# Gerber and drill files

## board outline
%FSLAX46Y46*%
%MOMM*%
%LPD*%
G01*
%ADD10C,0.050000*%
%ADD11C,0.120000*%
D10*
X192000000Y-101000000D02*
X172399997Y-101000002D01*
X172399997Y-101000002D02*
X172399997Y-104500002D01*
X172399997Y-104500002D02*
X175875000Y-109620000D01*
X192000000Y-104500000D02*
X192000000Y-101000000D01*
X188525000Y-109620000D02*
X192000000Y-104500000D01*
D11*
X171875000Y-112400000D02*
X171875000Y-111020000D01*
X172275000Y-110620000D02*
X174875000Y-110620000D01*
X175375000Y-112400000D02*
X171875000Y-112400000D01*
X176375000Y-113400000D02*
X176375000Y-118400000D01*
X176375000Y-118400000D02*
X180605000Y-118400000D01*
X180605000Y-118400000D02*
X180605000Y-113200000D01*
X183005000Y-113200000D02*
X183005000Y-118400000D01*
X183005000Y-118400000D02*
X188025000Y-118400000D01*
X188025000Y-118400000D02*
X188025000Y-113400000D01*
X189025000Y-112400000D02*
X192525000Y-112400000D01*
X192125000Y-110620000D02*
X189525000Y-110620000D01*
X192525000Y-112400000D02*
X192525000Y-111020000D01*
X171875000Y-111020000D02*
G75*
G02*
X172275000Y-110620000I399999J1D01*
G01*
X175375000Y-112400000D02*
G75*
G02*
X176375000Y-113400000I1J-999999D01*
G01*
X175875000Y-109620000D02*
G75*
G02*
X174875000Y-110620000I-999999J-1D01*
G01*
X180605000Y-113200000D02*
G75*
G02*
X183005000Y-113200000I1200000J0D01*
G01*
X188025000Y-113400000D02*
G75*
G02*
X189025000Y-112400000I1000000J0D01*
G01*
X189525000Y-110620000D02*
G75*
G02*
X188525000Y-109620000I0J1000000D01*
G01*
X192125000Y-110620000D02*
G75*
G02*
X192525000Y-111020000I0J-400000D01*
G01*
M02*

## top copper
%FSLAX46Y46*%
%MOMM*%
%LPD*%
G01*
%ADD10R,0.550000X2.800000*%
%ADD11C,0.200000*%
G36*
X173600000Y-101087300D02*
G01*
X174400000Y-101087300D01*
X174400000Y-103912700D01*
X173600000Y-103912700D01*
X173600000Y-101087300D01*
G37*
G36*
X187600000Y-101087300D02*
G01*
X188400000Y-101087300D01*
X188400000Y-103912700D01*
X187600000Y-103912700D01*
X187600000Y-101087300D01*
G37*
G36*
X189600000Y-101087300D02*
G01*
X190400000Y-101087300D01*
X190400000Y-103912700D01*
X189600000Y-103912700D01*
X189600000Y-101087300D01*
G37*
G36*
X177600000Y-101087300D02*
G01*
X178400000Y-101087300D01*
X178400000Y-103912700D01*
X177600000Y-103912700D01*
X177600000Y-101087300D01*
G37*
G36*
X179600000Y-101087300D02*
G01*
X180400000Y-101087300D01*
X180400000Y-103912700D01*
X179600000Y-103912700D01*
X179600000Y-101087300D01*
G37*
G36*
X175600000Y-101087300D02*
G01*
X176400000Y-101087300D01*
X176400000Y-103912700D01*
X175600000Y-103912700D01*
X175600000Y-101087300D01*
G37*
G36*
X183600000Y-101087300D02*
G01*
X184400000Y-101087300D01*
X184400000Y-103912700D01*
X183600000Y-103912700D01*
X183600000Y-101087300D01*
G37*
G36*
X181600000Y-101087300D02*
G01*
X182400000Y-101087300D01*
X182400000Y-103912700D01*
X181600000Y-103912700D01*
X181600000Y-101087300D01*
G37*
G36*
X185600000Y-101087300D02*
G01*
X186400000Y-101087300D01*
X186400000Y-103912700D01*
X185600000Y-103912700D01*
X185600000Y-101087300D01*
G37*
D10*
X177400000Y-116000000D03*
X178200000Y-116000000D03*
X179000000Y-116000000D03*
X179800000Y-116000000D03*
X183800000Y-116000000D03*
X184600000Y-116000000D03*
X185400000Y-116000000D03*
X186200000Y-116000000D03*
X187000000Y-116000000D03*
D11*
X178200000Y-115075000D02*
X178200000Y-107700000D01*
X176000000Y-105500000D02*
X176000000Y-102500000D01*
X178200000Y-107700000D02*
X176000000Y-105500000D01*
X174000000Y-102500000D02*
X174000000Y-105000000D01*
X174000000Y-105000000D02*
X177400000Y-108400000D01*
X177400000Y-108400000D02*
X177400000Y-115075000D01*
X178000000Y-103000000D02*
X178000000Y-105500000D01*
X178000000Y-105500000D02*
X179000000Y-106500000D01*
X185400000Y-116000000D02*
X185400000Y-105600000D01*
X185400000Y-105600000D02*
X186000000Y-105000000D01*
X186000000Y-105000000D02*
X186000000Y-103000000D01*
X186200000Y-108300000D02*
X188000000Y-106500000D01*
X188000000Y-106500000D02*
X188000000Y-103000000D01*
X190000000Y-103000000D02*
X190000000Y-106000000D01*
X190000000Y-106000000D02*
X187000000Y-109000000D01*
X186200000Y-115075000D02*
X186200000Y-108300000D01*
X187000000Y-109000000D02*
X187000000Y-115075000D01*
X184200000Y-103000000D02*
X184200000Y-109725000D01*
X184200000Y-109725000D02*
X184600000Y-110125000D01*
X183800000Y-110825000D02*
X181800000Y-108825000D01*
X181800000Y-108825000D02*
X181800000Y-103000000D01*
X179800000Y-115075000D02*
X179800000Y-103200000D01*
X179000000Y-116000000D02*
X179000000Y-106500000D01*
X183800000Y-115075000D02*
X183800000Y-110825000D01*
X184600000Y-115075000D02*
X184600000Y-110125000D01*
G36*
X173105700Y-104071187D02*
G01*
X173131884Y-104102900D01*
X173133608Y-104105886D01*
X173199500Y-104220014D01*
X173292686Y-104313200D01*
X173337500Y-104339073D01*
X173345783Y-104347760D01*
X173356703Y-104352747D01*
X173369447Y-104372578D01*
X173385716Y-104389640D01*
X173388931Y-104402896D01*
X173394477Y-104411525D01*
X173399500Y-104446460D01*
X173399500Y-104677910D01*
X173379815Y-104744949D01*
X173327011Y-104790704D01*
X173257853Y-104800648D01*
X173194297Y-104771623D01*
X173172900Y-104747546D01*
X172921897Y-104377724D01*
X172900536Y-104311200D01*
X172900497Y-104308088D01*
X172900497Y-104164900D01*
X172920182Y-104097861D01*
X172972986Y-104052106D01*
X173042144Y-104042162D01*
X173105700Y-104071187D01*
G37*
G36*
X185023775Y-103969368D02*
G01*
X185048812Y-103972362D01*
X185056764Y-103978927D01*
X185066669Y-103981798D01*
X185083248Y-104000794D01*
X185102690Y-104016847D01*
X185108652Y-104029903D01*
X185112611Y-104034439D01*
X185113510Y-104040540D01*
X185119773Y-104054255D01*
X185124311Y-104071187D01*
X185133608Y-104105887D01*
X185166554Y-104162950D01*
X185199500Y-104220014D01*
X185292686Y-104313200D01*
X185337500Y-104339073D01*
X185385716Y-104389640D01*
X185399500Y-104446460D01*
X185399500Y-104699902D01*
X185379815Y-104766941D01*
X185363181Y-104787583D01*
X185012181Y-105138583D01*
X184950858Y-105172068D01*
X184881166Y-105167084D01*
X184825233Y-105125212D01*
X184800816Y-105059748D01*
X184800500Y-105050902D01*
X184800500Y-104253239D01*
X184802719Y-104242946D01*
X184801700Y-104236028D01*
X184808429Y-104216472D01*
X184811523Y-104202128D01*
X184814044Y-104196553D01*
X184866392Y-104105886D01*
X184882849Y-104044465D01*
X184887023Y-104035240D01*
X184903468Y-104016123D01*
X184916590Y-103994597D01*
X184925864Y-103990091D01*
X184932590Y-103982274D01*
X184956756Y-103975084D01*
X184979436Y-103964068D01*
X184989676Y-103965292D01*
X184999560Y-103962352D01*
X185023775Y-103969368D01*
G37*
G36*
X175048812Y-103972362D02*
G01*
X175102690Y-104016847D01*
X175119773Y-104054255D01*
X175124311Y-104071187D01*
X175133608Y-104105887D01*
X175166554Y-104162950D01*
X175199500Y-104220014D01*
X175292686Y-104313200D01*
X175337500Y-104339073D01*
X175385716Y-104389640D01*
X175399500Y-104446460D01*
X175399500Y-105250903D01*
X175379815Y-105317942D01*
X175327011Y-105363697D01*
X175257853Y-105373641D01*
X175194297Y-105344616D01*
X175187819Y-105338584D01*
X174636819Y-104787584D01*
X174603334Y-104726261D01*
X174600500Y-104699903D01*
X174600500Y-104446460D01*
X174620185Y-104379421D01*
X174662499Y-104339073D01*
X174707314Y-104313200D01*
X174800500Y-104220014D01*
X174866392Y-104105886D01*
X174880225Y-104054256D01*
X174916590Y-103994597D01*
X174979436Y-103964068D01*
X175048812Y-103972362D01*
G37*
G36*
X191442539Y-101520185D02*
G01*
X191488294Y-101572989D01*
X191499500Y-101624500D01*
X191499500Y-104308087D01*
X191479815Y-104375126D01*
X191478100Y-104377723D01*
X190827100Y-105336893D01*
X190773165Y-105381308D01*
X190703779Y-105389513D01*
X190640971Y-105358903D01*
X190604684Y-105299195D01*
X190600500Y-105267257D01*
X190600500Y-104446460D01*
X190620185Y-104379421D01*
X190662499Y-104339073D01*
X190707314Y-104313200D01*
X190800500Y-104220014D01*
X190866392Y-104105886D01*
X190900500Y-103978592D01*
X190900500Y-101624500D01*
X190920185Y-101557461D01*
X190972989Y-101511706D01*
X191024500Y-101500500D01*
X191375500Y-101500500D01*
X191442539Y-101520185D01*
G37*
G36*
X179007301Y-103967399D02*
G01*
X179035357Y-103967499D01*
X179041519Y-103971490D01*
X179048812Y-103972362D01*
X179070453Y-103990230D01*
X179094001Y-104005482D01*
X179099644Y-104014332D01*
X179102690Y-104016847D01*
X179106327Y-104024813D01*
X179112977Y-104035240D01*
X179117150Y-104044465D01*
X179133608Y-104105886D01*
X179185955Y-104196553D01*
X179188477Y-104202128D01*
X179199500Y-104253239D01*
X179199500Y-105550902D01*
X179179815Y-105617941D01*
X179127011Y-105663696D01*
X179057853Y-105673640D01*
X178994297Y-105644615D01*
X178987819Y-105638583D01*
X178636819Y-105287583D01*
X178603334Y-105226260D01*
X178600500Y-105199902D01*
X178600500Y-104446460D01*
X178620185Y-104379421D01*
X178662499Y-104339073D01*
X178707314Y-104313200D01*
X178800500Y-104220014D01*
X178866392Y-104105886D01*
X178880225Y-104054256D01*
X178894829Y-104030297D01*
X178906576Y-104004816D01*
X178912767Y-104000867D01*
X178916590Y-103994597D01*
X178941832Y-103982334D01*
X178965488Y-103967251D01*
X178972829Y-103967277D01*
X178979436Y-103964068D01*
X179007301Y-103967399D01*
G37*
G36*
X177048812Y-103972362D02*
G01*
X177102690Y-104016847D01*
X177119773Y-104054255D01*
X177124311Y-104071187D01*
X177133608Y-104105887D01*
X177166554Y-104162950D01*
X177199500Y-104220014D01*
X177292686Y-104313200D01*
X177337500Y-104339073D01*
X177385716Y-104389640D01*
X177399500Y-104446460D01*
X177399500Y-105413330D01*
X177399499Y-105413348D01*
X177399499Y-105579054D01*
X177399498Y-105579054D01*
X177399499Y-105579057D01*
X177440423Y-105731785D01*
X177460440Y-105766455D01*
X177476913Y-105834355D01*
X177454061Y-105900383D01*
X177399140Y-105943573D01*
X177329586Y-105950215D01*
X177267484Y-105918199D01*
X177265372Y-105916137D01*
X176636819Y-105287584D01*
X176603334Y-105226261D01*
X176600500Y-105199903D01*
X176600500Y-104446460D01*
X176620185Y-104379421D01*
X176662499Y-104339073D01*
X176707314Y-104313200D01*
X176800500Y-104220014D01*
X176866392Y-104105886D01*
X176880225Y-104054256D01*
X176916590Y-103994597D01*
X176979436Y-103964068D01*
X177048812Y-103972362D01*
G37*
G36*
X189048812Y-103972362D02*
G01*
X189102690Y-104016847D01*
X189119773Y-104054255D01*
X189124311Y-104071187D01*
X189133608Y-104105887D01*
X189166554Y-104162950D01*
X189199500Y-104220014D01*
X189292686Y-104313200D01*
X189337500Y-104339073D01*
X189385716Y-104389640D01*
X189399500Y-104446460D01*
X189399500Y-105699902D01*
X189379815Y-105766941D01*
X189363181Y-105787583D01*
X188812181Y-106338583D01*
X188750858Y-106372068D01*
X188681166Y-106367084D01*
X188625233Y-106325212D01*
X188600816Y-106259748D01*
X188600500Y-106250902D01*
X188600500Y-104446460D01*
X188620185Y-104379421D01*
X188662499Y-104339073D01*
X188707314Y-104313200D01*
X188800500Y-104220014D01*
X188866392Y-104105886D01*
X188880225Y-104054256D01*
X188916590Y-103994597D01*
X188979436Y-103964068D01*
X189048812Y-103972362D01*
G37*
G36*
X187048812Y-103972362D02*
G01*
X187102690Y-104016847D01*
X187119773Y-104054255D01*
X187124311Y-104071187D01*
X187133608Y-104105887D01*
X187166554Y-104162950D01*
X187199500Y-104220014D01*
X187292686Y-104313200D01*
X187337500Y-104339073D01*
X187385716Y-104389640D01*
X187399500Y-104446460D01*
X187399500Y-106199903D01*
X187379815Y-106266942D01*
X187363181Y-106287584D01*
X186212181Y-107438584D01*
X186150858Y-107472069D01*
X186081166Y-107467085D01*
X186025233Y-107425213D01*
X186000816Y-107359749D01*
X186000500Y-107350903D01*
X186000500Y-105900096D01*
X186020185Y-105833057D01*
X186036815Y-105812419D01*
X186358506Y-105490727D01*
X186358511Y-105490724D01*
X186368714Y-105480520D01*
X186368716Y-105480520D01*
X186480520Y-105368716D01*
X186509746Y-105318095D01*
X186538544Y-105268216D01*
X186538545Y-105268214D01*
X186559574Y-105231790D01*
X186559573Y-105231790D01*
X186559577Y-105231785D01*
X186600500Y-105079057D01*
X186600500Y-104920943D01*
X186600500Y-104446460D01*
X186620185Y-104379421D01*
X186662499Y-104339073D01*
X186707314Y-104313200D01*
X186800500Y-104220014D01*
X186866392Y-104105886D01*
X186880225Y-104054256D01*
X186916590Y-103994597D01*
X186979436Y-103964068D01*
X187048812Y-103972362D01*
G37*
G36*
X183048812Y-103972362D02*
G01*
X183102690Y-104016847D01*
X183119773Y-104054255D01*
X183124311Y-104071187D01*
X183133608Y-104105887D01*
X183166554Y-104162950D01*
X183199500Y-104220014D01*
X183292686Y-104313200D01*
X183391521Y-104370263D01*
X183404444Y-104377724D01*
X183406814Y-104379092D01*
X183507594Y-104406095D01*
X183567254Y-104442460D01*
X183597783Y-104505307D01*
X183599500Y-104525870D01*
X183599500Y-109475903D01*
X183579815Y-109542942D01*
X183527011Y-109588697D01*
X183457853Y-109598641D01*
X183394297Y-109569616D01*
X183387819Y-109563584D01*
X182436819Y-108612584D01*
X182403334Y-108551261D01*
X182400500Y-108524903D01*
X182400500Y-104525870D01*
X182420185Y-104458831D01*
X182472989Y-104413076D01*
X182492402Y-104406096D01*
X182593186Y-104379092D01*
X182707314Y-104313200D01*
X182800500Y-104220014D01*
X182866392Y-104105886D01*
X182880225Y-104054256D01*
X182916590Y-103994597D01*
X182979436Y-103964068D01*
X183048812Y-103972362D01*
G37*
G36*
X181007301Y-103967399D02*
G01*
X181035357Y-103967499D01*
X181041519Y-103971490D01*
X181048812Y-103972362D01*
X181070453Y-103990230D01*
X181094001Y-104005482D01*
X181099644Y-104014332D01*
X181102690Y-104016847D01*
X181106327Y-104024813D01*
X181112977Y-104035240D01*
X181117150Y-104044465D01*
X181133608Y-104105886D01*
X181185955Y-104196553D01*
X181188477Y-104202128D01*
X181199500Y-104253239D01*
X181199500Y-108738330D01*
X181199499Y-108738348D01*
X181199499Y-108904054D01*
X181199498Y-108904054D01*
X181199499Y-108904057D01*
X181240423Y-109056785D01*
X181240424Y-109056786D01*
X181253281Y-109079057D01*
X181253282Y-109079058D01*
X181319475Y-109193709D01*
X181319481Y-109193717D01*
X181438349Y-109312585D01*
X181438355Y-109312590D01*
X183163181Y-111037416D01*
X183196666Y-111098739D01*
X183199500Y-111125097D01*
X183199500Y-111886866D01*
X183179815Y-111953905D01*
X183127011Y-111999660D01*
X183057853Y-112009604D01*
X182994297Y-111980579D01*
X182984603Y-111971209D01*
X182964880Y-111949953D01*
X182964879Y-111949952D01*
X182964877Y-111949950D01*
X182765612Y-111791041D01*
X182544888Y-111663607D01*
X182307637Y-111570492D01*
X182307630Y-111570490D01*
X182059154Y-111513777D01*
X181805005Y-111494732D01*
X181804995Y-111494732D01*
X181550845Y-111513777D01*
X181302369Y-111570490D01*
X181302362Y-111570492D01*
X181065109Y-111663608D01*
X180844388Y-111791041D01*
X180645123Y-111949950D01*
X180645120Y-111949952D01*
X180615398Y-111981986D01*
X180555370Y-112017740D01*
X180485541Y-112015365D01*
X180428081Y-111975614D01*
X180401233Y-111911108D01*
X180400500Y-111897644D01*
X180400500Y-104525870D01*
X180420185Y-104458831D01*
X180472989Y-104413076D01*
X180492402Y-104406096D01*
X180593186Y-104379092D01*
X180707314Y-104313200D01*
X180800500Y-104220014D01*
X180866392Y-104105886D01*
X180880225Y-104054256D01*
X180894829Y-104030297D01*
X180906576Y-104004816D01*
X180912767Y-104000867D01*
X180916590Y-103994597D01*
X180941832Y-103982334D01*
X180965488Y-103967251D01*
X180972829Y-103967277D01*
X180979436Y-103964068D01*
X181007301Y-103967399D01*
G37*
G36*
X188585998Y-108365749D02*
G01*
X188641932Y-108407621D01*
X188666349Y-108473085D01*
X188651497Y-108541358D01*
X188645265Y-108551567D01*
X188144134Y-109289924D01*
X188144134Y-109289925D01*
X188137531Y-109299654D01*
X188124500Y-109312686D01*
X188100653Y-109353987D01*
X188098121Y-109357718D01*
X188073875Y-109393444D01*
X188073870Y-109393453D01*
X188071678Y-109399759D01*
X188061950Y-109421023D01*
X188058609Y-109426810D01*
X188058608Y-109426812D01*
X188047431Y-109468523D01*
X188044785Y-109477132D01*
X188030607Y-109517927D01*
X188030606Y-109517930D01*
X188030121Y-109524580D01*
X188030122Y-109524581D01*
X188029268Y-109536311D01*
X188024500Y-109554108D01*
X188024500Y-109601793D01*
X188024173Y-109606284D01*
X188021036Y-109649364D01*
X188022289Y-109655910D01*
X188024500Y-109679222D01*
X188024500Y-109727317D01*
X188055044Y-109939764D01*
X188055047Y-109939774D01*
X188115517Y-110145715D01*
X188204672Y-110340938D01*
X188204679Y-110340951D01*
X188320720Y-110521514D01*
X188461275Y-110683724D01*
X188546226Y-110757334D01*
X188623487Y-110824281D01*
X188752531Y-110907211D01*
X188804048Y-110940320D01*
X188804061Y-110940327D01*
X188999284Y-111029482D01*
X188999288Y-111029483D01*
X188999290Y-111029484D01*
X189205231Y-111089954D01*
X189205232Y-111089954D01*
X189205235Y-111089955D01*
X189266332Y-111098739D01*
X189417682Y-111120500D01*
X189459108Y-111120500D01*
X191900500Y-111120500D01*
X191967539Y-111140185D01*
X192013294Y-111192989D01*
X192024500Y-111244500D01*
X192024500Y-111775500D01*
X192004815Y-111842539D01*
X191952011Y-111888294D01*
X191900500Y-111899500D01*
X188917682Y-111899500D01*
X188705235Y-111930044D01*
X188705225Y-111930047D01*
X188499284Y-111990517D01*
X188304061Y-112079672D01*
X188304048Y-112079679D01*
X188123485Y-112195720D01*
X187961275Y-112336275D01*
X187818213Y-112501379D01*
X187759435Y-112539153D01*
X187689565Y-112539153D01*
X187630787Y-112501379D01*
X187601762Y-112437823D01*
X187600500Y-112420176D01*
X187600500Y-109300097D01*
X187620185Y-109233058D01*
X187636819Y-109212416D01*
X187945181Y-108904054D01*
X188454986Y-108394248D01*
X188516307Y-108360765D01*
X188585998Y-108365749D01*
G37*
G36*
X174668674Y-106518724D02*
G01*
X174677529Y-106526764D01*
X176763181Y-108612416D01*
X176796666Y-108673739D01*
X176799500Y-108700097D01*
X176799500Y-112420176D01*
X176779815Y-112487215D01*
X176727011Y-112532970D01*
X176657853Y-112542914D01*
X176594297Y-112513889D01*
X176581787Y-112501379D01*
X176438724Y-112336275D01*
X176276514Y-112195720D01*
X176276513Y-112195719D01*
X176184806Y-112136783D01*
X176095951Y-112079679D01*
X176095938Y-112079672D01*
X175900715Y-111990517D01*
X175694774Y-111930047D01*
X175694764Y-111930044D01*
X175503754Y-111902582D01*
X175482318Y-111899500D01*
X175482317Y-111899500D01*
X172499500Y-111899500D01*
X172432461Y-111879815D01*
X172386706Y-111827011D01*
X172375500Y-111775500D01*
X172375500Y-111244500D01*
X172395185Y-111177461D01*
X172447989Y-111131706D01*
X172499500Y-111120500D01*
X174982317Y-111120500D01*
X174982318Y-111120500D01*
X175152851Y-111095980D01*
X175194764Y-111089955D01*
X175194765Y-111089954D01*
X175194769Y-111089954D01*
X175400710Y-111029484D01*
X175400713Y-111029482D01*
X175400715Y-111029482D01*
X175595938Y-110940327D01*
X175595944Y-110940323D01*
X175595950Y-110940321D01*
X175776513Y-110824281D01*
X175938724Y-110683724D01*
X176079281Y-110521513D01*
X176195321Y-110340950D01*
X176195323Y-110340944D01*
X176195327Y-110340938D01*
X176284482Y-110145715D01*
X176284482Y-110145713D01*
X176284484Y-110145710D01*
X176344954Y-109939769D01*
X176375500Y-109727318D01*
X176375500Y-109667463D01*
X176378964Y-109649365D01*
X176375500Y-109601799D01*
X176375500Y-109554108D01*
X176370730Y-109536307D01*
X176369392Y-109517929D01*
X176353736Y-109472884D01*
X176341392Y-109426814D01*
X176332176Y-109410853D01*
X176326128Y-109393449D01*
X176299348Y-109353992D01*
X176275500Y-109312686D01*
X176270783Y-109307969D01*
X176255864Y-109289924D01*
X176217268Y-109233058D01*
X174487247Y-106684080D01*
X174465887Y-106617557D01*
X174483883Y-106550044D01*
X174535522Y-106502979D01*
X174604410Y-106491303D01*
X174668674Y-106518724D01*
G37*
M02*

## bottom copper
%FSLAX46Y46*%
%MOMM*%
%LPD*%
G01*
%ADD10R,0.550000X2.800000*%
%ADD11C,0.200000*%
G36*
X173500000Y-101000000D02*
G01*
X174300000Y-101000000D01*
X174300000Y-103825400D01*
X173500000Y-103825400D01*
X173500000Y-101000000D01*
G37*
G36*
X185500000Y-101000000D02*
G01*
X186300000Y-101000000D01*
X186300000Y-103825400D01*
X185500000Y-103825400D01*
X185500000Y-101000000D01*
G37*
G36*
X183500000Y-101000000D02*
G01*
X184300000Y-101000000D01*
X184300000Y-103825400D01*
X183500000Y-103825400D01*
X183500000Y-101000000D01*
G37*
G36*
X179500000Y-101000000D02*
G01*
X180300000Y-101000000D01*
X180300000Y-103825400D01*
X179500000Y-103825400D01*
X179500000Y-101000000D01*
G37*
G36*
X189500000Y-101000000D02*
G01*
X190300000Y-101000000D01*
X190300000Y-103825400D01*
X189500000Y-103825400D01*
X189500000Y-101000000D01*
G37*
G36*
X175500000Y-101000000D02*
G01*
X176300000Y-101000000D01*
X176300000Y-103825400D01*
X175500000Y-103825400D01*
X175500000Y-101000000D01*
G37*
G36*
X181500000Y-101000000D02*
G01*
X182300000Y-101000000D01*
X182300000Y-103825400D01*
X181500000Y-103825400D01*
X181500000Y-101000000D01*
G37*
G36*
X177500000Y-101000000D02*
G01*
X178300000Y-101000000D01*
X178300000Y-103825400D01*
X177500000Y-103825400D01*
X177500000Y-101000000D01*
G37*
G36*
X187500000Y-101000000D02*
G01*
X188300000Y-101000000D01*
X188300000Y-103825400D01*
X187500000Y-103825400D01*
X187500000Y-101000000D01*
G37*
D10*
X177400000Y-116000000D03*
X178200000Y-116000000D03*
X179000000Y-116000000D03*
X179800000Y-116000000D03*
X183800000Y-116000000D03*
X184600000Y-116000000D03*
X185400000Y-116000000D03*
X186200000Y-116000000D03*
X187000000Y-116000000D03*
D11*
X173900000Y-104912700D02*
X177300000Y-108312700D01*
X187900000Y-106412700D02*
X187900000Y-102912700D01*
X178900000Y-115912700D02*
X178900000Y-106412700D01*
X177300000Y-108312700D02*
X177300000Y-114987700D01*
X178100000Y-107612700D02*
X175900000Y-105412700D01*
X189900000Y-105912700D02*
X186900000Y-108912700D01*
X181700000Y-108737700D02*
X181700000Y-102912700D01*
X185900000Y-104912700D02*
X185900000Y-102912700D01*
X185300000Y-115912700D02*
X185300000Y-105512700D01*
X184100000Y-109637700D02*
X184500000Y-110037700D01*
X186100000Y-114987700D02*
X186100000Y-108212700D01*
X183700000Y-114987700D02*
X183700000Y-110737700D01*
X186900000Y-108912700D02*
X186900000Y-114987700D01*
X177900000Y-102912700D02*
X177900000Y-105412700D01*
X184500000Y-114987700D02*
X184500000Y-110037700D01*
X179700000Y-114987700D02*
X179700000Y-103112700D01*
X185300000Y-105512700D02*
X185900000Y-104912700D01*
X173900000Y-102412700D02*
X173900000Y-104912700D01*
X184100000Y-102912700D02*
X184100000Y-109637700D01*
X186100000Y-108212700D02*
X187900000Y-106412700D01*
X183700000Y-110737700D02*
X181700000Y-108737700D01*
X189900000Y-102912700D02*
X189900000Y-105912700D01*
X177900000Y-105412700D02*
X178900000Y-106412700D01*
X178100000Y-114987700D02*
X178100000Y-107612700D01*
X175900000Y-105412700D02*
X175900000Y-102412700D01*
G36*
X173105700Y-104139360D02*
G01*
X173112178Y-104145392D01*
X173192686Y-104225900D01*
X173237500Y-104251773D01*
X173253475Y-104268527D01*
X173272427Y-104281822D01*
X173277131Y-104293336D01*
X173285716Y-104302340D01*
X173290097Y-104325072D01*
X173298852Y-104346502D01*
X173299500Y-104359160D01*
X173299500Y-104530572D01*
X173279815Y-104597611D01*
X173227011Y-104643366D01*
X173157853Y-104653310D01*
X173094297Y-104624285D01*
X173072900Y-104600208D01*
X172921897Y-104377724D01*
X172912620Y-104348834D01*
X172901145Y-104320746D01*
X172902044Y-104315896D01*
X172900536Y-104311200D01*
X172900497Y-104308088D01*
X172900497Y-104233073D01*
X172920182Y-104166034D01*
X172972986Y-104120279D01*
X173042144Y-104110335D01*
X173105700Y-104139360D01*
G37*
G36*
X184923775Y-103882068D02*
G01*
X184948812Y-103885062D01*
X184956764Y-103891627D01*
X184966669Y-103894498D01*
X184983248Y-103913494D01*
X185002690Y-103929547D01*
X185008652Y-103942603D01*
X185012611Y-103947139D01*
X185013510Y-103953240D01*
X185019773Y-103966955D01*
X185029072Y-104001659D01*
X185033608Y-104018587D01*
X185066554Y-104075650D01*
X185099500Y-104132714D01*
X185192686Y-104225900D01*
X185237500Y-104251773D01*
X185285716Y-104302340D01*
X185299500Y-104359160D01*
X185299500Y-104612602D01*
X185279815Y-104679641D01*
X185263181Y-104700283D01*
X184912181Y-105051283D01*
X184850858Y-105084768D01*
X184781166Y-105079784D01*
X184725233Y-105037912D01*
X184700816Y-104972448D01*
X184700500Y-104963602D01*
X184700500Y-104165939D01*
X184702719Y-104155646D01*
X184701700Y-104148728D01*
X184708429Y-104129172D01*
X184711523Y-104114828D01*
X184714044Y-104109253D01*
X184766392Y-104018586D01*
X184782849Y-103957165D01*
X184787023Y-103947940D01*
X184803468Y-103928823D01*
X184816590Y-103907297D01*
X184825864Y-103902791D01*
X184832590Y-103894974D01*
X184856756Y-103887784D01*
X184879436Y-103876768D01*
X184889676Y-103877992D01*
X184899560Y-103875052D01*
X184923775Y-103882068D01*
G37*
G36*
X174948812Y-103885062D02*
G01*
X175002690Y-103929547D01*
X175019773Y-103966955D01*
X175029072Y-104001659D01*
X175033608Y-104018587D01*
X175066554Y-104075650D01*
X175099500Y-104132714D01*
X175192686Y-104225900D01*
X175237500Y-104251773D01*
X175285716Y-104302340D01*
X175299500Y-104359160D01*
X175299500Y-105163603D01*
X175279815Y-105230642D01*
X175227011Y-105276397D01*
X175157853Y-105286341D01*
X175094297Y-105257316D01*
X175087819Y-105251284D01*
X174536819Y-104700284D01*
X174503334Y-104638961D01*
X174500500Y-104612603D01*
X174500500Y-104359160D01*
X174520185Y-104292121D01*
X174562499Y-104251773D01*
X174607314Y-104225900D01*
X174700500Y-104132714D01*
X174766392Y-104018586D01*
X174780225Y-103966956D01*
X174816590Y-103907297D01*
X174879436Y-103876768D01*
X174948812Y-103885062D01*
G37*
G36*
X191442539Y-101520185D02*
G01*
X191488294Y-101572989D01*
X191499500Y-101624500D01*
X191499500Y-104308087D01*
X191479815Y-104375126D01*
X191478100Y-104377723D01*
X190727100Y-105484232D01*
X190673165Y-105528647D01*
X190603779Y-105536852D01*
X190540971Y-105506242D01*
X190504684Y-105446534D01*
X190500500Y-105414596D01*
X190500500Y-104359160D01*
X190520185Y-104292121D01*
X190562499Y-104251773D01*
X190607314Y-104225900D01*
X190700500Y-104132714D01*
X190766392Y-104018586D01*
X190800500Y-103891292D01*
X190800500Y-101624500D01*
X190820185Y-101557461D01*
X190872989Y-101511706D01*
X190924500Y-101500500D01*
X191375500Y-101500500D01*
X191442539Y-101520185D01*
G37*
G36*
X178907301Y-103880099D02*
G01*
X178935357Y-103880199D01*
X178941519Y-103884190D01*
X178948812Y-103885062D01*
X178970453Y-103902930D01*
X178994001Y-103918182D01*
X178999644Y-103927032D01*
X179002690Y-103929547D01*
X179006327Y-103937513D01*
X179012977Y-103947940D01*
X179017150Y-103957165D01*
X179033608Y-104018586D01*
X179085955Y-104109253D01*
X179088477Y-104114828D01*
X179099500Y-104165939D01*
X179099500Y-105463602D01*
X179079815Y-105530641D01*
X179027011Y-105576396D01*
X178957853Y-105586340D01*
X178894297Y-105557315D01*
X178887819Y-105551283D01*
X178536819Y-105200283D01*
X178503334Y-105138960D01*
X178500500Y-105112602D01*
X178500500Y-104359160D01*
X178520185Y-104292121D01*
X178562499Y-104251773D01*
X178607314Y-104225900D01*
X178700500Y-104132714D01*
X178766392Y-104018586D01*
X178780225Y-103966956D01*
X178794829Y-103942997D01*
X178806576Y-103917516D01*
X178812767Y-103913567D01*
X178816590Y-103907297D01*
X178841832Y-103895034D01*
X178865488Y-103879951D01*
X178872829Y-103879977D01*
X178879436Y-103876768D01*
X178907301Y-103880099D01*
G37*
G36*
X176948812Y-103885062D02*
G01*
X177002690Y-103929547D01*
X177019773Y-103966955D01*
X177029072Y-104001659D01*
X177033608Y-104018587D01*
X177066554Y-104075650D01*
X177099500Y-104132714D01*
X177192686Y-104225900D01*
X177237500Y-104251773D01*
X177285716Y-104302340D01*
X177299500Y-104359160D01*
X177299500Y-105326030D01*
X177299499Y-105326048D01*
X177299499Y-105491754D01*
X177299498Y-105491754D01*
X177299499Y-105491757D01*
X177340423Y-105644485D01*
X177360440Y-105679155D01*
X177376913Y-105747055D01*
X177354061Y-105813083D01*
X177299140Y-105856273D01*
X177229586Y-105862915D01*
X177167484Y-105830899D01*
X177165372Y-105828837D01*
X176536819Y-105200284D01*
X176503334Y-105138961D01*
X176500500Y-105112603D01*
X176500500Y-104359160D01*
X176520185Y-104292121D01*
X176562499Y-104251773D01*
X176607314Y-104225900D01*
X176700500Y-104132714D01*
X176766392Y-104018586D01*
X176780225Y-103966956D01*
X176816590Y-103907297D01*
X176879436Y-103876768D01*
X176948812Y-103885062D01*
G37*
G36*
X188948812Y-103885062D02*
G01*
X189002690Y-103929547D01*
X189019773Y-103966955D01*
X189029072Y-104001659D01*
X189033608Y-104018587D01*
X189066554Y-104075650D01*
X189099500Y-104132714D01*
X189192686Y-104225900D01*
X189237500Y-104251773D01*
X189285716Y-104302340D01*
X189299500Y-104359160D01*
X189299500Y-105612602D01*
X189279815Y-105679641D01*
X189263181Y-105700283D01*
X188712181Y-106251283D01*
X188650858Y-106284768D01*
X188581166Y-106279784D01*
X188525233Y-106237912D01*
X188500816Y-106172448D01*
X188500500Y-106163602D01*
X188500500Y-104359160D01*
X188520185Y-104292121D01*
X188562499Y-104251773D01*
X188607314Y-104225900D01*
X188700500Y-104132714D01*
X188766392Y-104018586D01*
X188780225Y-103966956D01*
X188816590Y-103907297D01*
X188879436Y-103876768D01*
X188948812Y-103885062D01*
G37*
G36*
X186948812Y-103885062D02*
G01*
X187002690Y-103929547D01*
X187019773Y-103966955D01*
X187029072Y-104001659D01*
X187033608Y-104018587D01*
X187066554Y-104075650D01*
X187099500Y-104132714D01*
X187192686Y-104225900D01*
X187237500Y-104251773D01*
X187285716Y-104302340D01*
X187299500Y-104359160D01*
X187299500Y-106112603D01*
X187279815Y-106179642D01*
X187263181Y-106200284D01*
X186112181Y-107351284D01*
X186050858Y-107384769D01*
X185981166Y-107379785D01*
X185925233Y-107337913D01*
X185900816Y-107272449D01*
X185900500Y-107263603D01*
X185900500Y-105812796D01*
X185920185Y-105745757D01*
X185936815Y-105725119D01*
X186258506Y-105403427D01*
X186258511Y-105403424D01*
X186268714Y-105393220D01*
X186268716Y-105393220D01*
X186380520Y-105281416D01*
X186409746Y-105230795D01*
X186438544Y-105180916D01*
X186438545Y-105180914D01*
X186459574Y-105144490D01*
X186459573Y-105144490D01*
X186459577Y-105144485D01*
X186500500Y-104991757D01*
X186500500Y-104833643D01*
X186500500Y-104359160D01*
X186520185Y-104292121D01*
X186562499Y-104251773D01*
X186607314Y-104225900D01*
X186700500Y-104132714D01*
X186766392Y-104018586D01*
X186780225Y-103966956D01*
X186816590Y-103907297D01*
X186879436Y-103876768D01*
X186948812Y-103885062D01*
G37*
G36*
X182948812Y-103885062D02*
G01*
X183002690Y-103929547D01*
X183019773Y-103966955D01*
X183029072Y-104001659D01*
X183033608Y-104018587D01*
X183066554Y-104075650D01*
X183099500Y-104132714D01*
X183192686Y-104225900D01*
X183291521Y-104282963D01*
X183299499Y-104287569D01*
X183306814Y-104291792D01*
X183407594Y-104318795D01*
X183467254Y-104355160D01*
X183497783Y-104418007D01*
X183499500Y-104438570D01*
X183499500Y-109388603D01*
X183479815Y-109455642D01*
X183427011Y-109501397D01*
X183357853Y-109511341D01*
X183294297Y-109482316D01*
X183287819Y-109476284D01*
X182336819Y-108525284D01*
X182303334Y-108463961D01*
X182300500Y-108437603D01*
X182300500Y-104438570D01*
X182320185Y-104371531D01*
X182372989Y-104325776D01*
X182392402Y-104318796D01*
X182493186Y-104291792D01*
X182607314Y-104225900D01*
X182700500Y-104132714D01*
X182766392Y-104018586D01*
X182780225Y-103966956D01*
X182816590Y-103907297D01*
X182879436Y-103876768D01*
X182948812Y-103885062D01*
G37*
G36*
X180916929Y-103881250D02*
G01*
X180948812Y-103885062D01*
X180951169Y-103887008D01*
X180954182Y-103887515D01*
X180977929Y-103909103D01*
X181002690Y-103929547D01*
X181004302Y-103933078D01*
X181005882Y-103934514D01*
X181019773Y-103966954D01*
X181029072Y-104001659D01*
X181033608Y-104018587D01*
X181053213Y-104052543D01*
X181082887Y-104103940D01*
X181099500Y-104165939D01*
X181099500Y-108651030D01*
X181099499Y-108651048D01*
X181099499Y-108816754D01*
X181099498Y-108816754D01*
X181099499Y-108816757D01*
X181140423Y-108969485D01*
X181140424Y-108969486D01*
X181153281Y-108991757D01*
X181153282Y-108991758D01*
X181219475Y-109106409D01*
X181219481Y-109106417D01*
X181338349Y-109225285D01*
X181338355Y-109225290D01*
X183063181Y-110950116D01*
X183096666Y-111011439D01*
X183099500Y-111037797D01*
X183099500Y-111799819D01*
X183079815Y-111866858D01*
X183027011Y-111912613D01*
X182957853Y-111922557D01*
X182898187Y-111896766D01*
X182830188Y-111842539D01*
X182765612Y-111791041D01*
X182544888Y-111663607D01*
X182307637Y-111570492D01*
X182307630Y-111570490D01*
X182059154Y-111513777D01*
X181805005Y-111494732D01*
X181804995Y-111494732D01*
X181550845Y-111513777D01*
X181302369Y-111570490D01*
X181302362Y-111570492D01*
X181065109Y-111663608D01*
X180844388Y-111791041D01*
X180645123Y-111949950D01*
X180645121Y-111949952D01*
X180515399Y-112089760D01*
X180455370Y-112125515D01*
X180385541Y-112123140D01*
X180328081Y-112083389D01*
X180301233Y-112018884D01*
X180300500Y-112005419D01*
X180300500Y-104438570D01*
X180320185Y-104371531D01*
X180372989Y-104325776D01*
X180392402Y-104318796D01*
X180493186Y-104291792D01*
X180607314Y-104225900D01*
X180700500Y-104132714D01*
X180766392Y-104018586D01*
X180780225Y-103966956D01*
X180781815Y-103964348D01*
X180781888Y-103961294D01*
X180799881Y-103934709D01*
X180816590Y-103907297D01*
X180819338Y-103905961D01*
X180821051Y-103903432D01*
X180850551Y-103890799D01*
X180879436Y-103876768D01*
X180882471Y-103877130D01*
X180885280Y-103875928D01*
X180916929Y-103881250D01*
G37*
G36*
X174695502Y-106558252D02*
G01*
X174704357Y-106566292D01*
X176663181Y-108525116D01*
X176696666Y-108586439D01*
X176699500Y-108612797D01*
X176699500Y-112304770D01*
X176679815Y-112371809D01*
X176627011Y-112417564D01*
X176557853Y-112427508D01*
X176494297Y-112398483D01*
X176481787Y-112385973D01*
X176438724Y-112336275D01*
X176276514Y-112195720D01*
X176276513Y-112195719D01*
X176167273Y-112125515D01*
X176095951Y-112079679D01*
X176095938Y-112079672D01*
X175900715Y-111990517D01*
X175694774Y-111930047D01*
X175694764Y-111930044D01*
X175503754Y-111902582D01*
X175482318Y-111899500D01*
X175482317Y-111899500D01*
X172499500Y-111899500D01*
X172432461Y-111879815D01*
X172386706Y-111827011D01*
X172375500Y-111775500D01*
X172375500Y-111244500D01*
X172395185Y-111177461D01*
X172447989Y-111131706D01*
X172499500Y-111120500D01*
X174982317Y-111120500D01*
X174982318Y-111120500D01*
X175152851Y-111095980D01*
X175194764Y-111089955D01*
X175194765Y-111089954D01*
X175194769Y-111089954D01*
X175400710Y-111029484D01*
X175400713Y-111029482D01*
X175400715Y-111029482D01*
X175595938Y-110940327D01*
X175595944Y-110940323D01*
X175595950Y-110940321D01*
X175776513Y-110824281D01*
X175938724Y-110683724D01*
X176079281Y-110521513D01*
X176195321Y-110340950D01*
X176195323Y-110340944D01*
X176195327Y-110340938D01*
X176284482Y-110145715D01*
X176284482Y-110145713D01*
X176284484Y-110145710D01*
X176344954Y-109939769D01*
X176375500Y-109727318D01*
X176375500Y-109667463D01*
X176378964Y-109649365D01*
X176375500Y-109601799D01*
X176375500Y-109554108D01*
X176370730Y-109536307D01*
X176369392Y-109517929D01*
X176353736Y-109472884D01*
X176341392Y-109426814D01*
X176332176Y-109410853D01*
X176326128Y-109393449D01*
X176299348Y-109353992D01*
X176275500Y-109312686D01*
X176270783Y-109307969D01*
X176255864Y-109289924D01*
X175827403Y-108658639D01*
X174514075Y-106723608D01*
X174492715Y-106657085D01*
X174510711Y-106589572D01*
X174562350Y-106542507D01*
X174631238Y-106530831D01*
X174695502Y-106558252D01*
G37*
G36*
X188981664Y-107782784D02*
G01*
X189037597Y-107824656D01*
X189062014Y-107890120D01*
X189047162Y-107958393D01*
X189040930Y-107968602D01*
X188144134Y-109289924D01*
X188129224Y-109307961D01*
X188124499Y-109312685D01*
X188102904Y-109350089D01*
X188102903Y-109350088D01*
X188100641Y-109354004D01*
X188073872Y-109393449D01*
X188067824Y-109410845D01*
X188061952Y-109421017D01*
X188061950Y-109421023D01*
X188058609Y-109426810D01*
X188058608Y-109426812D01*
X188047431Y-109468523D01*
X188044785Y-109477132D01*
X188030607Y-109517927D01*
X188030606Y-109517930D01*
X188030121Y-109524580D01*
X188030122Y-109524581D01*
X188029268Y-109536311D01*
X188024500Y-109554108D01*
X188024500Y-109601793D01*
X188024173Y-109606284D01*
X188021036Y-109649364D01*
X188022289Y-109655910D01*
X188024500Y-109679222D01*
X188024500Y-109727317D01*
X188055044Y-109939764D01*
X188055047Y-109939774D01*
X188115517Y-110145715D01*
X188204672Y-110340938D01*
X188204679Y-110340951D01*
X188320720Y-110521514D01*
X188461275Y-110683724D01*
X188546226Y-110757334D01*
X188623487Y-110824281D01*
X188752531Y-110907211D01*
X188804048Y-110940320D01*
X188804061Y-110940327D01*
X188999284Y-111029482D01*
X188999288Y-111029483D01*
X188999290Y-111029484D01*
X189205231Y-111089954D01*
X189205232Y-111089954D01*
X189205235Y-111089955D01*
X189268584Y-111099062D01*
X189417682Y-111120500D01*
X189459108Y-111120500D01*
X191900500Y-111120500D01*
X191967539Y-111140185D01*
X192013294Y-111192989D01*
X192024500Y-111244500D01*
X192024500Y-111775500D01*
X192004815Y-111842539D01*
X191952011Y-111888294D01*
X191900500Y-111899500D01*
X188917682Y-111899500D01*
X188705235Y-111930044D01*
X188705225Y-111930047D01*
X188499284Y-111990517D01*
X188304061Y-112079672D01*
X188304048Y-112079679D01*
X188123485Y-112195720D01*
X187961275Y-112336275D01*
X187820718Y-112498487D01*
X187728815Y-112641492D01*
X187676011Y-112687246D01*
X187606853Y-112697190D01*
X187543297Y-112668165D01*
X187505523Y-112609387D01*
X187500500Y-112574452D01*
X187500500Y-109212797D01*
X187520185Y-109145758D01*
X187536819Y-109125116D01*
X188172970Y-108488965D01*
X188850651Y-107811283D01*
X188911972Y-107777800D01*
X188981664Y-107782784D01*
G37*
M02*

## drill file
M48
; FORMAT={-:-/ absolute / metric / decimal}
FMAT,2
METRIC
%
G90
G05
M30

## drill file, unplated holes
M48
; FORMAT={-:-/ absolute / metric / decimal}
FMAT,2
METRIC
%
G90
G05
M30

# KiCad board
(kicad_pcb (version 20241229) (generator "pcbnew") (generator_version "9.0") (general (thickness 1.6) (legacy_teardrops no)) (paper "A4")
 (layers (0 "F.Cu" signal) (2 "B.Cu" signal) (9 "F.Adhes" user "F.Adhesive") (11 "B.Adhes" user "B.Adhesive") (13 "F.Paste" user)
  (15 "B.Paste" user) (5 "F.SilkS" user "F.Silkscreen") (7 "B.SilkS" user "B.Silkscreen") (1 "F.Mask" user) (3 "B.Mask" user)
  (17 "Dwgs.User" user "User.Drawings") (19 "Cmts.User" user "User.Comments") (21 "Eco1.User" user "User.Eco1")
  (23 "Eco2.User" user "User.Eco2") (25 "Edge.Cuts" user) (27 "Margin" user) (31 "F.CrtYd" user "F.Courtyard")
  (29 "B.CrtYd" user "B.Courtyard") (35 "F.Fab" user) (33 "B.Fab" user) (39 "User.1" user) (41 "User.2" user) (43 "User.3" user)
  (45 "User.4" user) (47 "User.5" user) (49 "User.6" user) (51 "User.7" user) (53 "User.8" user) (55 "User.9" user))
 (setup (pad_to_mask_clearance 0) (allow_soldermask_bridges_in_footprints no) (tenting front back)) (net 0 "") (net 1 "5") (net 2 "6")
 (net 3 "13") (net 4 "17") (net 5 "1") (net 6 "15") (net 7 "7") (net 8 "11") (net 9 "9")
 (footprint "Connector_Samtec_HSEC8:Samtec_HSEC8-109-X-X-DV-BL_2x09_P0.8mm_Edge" (layer "F.Cu") (at 182.2 118.4)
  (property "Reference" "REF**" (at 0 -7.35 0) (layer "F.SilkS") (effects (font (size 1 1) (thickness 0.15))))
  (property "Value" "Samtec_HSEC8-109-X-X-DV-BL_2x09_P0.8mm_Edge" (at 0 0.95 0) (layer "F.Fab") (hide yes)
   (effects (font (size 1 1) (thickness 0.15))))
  (fp_line (start -10.325 -6) (end -10.325 -7.38) (stroke (width 0.12) (type solid)) (layer "Edge.Cuts"))
  (fp_line (start -9.925 -7.78) (end -7.325 -7.78) (stroke (width 0.12) (type solid)) (layer "Edge.Cuts"))
  (fp_line (start -6.825 -6) (end -10.325 -6) (stroke (width 0.12) (type solid)) (layer "Edge.Cuts"))
  (fp_line (start -5.825 -5) (end -5.825 0) (stroke (width 0.12) (type solid)) (layer "Edge.Cuts"))
  (fp_line (start -5.825 0) (end -1.595 0) (stroke (width 0.12) (type solid)) (layer "Edge.Cuts"))
  (fp_line (start -1.595 0) (end -1.595 -5.2) (stroke (width 0.12) (type solid)) (layer "Edge.Cuts"))
  (fp_line (start 0.805 -5.2) (end 0.805 0) (stroke (width 0.12) (type solid)) (layer "Edge.Cuts"))
  (fp_line (start 0.805 0) (end 5.825 0) (stroke (width 0.12) (type solid)) (layer "Edge.Cuts"))
  (fp_line (start 5.825 0) (end 5.825 -5) (stroke (width 0.12) (type solid)) (layer "Edge.Cuts"))
  (fp_line (start 6.825 -6) (end 10.325 -6) (stroke (width 0.12) (type solid)) (layer "Edge.Cuts"))
  (fp_line (start 9.925 -7.78) (end 7.325 -7.78) (stroke (width 0.12) (type solid)) (layer "Edge.Cuts"))
  (fp_line (start 10.325 -6) (end 10.325 -7.38) (stroke (width 0.12) (type solid)) (layer "Edge.Cuts"))
  (fp_arc (start -10.325 -7.38) (mid -10.207843 -7.662843) (end -9.925 -7.78) (stroke (width 0.12) (type solid)) (layer "Edge.Cuts"))
  (fp_arc (start -6.825 -6) (mid -6.117893 -5.707107) (end -5.825 -5) (stroke (width 0.12) (type solid)) (layer "Edge.Cuts"))
  (fp_arc (start -6.325 -8.78) (mid -6.617893 -8.072893) (end -7.325 -7.78) (stroke (width 0.12) (type solid)) (layer "Edge.Cuts"))
  (fp_arc (start -1.595 -5.2) (mid -0.395 -6.4) (end 0.805 -5.2) (stroke (width 0.12) (type solid)) (layer "Edge.Cuts"))
  (fp_arc (start 5.825 -5) (mid 6.117893 -5.707107) (end 6.825 -6) (stroke (width 0.12) (type solid)) (layer "Edge.Cuts"))
  (fp_arc (start 7.325 -7.78) (mid 6.617893 -8.072893) (end 6.325 -8.78) (stroke (width 0.12) (type solid)) (layer "Edge.Cuts"))
  (fp_arc (start 9.925 -7.78) (mid 10.207843 -7.662843) (end 10.325 -7.38) (stroke (width 0.12) (type solid)) (layer "Edge.Cuts"))
  (pad "1" connect rect (at -4.8 -2.4) (size 0.55 2.8) (layers "F.Cu" "F.Mask"))
  (pad "2" connect rect (at -4.8 -2.4) (size 0.55 2.8) (layers "B.Cu" "B.Mask"))
  (pad "3" connect rect (at -4 -2.4) (size 0.55 2.8) (layers "F.Cu" "F.Mask"))
  (pad "4" connect rect (at -4 -2.4) (size 0.55 2.8) (layers "B.Cu" "B.Mask"))
  (pad "5" connect rect (at -3.2 -2.4) (size 0.55 2.8) (layers "F.Cu" "F.Mask") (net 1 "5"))
  (pad "6" connect rect (at -3.2 -2.4) (size 0.55 2.8) (layers "B.Cu" "B.Mask") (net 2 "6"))
  (pad "7" connect rect (at -2.4 -2.4) (size 0.55 2.8) (layers "F.Cu" "F.Mask"))
  (pad "8" connect rect (at -2.4 -2.4) (size 0.55 2.8) (layers "B.Cu" "B.Mask"))
  (pad "9" connect rect (at 1.6 -2.4) (size 0.55 2.8) (layers "F.Cu" "F.Mask"))
  (pad "10" connect rect (at 1.6 -2.4) (size 0.55 2.8) (layers "B.Cu" "B.Mask"))
  (pad "11" connect rect (at 2.4 -2.4) (size 0.55 2.8) (layers "F.Cu" "F.Mask"))
  (pad "12" connect rect (at 2.4 -2.4) (size 0.55 2.8) (layers "B.Cu" "B.Mask"))
  (pad "13" connect rect (at 3.2 -2.4) (size 0.55 2.8) (layers "F.Cu" "F.Mask") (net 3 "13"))
  (pad "14" connect rect (at 3.2 -2.4) (size 0.55 2.8) (layers "B.Cu" "B.Mask"))
  (pad "15" connect rect (at 4 -2.4) (size 0.55 2.8) (layers "F.Cu" "F.Mask"))
  (pad "16" connect rect (at 4 -2.4) (size 0.55 2.8) (layers "B.Cu" "B.Mask"))
  (pad "17" connect rect (at 4.8 -2.4) (size 0.55 2.8) (layers "F.Cu" "F.Mask") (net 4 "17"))
  (pad "18" connect rect (at 4.8 -2.4) (size 0.55 2.8) (layers "B.Cu" "B.Mask")))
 (gr_rect (start 173.6 101.0873) (end 174.4 103.9127) (stroke (width 0) (type solid)) (fill yes) (layers "F.Cu" "F.Mask") (net 5))
 (gr_rect (start 187.6 101.0873) (end 188.4 103.9127) (stroke (width 0) (type solid)) (fill yes) (layers "F.Cu" "F.Mask") (net 6))
 (gr_rect (start 189.6 101.0873) (end 190.4 103.9127) (stroke (width 0) (type solid)) (fill yes) (layers "F.Cu" "F.Mask") (net 4))
 (gr_rect (start 177.6 101.0873) (end 178.4 103.9127) (stroke (width 0) (type solid)) (fill yes) (layers "F.Cu" "F.Mask") (net 1))
 (gr_rect (start 179.6 101.0873) (end 180.4 103.9127) (stroke (width 0) (type solid)) (fill yes) (layers "F.Cu" "F.Mask") (net 7))
 (gr_rect (start 175.6 101.0873) (end 176.4 103.9127) (stroke (width 0) (type solid)) (fill yes) (layers "F.Cu" "F.Mask") (net 5))
 (gr_rect (start 183.6 101.0873) (end 184.4 103.9127) (stroke (width 0) (type solid)) (fill yes) (layers "F.Cu" "F.Mask") (net 8))
 (gr_rect (start 181.6 101.0873) (end 182.4 103.9127) (stroke (width 0) (type solid)) (fill yes) (layers "F.Cu" "F.Mask") (net 9))
 (gr_rect (start 185.6 101.0873) (end 186.4 103.9127) (stroke (width 0) (type solid)) (fill yes) (layers "F.Cu" "F.Mask") (net 3))
 (gr_rect (start 175.5 101) (end 176.3 103.8254) (stroke (width 0) (type solid)) (fill yes) (layers "B.Cu" "B.Mask") (net 5))
 (gr_rect (start 177.5 101) (end 178.3 103.8254) (stroke (width 0) (type solid)) (fill yes) (layers "B.Cu" "B.Mask") (net 2))
 (gr_rect (start 173.5 101) (end 174.3 103.8254) (stroke (width 0) (type solid)) (fill yes) (layers "B.Cu" "B.Mask") (net 5))
 (gr_rect (start 179.5 101) (end 180.3 103.8254) (stroke (width 0) (type solid)) (fill yes) (layers "B.Cu" "B.Mask") (net 7))
 (gr_rect (start 189.5 101) (end 190.3 103.8254) (stroke (width 0) (type solid)) (fill yes) (layers "B.Cu" "B.Mask") (net 4))
 (gr_rect (start 183.5 101) (end 184.3 103.8254) (stroke (width 0) (type solid)) (fill yes) (layers "B.Cu" "B.Mask") (net 8))
 (gr_rect (start 181.5 101) (end 182.3 103.8254) (stroke (width 0) (type solid)) (fill yes) (layers "B.Cu" "B.Mask") (net 9))
 (gr_rect (start 187.5 101) (end 188.3 103.8254) (stroke (width 0) (type solid)) (fill yes) (layers "B.Cu" "B.Mask") (net 6))
 (gr_rect (start 185.5 101) (end 186.3 103.8254) (stroke (width 0) (type solid)) (fill yes) (layers "B.Cu" "B.Mask") (net 3))
 (gr_line (start 192 101) (end 172.399997 101.000002) (stroke (width 0.05) (type default)) (layer "Edge.Cuts"))
 (gr_line (start 172.399997 104.500002) (end 175.875 109.62) (stroke (width 0.05) (type solid)) (layer "Edge.Cuts"))
 (gr_line (start 172.399997 101.000002) (end 172.399997 104.500002) (stroke (width 0.05) (type default)) (layer "Edge.Cuts"))
 (gr_line (start 192 104.5) (end 192 101) (stroke (width 0.05) (type default)) (layer "Edge.Cuts"))
 (gr_line (start 188.525 109.62) (end 192 104.5) (stroke (width 0.05) (type default)) (layer "Edge.Cuts"))
 (segment (start 178.2 107.7) (end 176 105.5) (width 0.2) (layer "F.Cu") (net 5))
 (segment (start 176 105.5) (end 176 102.5) (width 0.2) (layer "F.Cu") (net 5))
 (segment (start 178.2 115.075) (end 178.2 107.7) (width 0.2) (layer "F.Cu") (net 5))
 (segment (start 177.4 108.4) (end 177.4 115.075) (width 0.2) (layer "F.Cu") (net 5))
 (segment (start 174 102.5) (end 174 105) (width 0.2) (layer "F.Cu") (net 5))
 (segment (start 174 105) (end 177.4 108.4) (width 0.2) (layer "F.Cu") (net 5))
 (segment (start 177.3 108.3127) (end 177.3 114.9877) (width 0.2) (layer "B.Cu") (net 5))
 (segment (start 175.9 105.4127) (end 175.9 102.4127) (width 0.2) (layer "B.Cu") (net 5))
 (segment (start 173.9 102.4127) (end 173.9 104.9127) (width 0.2) (layer "B.Cu") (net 5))
 (segment (start 178.1 114.9877) (end 178.1 107.6127) (width 0.2) (layer "B.Cu") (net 5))
 (segment (start 173.9 104.9127) (end 177.3 108.3127) (width 0.2) (layer "B.Cu") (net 5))
 (segment (start 178.1 107.6127) (end 175.9 105.4127) (width 0.2) (layer "B.Cu") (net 5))
 (segment (start 178 105.5) (end 179 106.5) (width 0.2) (layer "F.Cu") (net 1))
 (segment (start 178 103) (end 178 105.5) (width 0.2) (layer "F.Cu") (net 1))
 (segment (start 179 116) (end 179 106.5) (width 0.2) (layer "F.Cu") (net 1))
 (segment (start 179.8 115.075) (end 179.8 103.2) (width 0.2) (layer "F.Cu") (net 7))
 (segment (start 179.7 114.9877) (end 179.7 103.1127) (width 0.2) (layer "B.Cu") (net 7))
 (segment (start 183.8 115.075) (end 183.8 110.825) (width 0.2) (layer "F.Cu") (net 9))
 (segment (start 183.8 110.825) (end 181.8 108.825) (width 0.2) (layer "F.Cu") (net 9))
 (segment (start 181.8 108.825) (end 181.8 103) (width 0.2) (layer "F.Cu") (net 9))
 (segment (start 183.7 114.9877) (end 183.7 110.7377) (width 0.2) (layer "B.Cu") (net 9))
 (segment (start 181.7 108.7377) (end 181.7 102.9127) (width 0.2) (layer "B.Cu") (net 9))
 (segment (start 183.7 110.7377) (end 181.7 108.7377) (width 0.2) (layer "B.Cu") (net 9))
 (segment (start 184.6 115.075) (end 184.6 110.125) (width 0.2) (layer "F.Cu") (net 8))
 (segment (start 184.2 103) (end 184.2 109.725) (width 0.2) (layer "F.Cu") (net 8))
 (segment (start 184.2 109.725) (end 184.6 110.125) (width 0.2) (layer "F.Cu") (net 8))
 (segment (start 184.1 109.6377) (end 184.5 110.0377) (width 0.2) (layer "B.Cu") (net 8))
 (segment (start 184.5 114.9877) (end 184.5 110.0377) (width 0.2) (layer "B.Cu") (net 8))
 (segment (start 184.1 102.9127) (end 184.1 109.6377) (width 0.2) (layer "B.Cu") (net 8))
 (segment (start 185.4 105.6) (end 186 105) (width 0.2) (layer "F.Cu") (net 3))
 (segment (start 186 105) (end 186 103) (width 0.2) (layer "F.Cu") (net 3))
 (segment (start 185.4 116) (end 185.4 105.6) (width 0.2) (layer "F.Cu") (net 3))
 (segment (start 185.3 115.9127) (end 185.3 105.5127) (width 0.2) (layer "B.Cu") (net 3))
 (segment (start 185.3 105.5127) (end 185.9 104.9127) (width 0.2) (layer "B.Cu") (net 3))
 (segment (start 185.9 104.9127) (end 185.9 102.9127) (width 0.2) (layer "B.Cu") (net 3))
 (segment (start 188 106.5) (end 188 103) (width 0.2) (layer "F.Cu") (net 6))
 (segment (start 186.2 108.3) (end 188 106.5) (width 0.2) (layer "F.Cu") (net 6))
 (segment (start 186.2 115.075) (end 186.2 108.3) (width 0.2) (layer "F.Cu") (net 6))
 (segment (start 187.9 106.4127) (end 187.9 102.9127) (width 0.2) (layer "B.Cu") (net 6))
 (segment (start 186.1 114.9877) (end 186.1 108.2127) (width 0.2) (layer "B.Cu") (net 6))
 (segment (start 186.1 108.2127) (end 187.9 106.4127) (width 0.2) (layer "B.Cu") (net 6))
 (segment (start 190 106) (end 187 109) (width 0.2) (layer "F.Cu") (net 4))
 (segment (start 190 103) (end 190 106) (width 0.2) (layer "F.Cu") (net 4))
 (segment (start 187 109) (end 187 115.075) (width 0.2) (layer "F.Cu") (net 4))
 (segment (start 189.9 102.9127) (end 189.9 105.9127) (width 0.2) (layer "B.Cu") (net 4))
 (segment (start 189.9 105.9127) (end 186.9 108.9127) (width 0.2) (layer "B.Cu") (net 4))
 (segment (start 186.9 108.9127) (end 186.9 114.9877) (width 0.2) (layer "B.Cu") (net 4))
 (segment (start 177.9 105.4127) (end 178.9 106.4127) (width 0.2) (layer "B.Cu") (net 2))
 (segment (start 178.9 115.9127) (end 178.9 106.4127) (width 0.2) (layer "B.Cu") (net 2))
 (segment (start 177.9 102.9127) (end 177.9 105.4127) (width 0.2) (layer "B.Cu") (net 2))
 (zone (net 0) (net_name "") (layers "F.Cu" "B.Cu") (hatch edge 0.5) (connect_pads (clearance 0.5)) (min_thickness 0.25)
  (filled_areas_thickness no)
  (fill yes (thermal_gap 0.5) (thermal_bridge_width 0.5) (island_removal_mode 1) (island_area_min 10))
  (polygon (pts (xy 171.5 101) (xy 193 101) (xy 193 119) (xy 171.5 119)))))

